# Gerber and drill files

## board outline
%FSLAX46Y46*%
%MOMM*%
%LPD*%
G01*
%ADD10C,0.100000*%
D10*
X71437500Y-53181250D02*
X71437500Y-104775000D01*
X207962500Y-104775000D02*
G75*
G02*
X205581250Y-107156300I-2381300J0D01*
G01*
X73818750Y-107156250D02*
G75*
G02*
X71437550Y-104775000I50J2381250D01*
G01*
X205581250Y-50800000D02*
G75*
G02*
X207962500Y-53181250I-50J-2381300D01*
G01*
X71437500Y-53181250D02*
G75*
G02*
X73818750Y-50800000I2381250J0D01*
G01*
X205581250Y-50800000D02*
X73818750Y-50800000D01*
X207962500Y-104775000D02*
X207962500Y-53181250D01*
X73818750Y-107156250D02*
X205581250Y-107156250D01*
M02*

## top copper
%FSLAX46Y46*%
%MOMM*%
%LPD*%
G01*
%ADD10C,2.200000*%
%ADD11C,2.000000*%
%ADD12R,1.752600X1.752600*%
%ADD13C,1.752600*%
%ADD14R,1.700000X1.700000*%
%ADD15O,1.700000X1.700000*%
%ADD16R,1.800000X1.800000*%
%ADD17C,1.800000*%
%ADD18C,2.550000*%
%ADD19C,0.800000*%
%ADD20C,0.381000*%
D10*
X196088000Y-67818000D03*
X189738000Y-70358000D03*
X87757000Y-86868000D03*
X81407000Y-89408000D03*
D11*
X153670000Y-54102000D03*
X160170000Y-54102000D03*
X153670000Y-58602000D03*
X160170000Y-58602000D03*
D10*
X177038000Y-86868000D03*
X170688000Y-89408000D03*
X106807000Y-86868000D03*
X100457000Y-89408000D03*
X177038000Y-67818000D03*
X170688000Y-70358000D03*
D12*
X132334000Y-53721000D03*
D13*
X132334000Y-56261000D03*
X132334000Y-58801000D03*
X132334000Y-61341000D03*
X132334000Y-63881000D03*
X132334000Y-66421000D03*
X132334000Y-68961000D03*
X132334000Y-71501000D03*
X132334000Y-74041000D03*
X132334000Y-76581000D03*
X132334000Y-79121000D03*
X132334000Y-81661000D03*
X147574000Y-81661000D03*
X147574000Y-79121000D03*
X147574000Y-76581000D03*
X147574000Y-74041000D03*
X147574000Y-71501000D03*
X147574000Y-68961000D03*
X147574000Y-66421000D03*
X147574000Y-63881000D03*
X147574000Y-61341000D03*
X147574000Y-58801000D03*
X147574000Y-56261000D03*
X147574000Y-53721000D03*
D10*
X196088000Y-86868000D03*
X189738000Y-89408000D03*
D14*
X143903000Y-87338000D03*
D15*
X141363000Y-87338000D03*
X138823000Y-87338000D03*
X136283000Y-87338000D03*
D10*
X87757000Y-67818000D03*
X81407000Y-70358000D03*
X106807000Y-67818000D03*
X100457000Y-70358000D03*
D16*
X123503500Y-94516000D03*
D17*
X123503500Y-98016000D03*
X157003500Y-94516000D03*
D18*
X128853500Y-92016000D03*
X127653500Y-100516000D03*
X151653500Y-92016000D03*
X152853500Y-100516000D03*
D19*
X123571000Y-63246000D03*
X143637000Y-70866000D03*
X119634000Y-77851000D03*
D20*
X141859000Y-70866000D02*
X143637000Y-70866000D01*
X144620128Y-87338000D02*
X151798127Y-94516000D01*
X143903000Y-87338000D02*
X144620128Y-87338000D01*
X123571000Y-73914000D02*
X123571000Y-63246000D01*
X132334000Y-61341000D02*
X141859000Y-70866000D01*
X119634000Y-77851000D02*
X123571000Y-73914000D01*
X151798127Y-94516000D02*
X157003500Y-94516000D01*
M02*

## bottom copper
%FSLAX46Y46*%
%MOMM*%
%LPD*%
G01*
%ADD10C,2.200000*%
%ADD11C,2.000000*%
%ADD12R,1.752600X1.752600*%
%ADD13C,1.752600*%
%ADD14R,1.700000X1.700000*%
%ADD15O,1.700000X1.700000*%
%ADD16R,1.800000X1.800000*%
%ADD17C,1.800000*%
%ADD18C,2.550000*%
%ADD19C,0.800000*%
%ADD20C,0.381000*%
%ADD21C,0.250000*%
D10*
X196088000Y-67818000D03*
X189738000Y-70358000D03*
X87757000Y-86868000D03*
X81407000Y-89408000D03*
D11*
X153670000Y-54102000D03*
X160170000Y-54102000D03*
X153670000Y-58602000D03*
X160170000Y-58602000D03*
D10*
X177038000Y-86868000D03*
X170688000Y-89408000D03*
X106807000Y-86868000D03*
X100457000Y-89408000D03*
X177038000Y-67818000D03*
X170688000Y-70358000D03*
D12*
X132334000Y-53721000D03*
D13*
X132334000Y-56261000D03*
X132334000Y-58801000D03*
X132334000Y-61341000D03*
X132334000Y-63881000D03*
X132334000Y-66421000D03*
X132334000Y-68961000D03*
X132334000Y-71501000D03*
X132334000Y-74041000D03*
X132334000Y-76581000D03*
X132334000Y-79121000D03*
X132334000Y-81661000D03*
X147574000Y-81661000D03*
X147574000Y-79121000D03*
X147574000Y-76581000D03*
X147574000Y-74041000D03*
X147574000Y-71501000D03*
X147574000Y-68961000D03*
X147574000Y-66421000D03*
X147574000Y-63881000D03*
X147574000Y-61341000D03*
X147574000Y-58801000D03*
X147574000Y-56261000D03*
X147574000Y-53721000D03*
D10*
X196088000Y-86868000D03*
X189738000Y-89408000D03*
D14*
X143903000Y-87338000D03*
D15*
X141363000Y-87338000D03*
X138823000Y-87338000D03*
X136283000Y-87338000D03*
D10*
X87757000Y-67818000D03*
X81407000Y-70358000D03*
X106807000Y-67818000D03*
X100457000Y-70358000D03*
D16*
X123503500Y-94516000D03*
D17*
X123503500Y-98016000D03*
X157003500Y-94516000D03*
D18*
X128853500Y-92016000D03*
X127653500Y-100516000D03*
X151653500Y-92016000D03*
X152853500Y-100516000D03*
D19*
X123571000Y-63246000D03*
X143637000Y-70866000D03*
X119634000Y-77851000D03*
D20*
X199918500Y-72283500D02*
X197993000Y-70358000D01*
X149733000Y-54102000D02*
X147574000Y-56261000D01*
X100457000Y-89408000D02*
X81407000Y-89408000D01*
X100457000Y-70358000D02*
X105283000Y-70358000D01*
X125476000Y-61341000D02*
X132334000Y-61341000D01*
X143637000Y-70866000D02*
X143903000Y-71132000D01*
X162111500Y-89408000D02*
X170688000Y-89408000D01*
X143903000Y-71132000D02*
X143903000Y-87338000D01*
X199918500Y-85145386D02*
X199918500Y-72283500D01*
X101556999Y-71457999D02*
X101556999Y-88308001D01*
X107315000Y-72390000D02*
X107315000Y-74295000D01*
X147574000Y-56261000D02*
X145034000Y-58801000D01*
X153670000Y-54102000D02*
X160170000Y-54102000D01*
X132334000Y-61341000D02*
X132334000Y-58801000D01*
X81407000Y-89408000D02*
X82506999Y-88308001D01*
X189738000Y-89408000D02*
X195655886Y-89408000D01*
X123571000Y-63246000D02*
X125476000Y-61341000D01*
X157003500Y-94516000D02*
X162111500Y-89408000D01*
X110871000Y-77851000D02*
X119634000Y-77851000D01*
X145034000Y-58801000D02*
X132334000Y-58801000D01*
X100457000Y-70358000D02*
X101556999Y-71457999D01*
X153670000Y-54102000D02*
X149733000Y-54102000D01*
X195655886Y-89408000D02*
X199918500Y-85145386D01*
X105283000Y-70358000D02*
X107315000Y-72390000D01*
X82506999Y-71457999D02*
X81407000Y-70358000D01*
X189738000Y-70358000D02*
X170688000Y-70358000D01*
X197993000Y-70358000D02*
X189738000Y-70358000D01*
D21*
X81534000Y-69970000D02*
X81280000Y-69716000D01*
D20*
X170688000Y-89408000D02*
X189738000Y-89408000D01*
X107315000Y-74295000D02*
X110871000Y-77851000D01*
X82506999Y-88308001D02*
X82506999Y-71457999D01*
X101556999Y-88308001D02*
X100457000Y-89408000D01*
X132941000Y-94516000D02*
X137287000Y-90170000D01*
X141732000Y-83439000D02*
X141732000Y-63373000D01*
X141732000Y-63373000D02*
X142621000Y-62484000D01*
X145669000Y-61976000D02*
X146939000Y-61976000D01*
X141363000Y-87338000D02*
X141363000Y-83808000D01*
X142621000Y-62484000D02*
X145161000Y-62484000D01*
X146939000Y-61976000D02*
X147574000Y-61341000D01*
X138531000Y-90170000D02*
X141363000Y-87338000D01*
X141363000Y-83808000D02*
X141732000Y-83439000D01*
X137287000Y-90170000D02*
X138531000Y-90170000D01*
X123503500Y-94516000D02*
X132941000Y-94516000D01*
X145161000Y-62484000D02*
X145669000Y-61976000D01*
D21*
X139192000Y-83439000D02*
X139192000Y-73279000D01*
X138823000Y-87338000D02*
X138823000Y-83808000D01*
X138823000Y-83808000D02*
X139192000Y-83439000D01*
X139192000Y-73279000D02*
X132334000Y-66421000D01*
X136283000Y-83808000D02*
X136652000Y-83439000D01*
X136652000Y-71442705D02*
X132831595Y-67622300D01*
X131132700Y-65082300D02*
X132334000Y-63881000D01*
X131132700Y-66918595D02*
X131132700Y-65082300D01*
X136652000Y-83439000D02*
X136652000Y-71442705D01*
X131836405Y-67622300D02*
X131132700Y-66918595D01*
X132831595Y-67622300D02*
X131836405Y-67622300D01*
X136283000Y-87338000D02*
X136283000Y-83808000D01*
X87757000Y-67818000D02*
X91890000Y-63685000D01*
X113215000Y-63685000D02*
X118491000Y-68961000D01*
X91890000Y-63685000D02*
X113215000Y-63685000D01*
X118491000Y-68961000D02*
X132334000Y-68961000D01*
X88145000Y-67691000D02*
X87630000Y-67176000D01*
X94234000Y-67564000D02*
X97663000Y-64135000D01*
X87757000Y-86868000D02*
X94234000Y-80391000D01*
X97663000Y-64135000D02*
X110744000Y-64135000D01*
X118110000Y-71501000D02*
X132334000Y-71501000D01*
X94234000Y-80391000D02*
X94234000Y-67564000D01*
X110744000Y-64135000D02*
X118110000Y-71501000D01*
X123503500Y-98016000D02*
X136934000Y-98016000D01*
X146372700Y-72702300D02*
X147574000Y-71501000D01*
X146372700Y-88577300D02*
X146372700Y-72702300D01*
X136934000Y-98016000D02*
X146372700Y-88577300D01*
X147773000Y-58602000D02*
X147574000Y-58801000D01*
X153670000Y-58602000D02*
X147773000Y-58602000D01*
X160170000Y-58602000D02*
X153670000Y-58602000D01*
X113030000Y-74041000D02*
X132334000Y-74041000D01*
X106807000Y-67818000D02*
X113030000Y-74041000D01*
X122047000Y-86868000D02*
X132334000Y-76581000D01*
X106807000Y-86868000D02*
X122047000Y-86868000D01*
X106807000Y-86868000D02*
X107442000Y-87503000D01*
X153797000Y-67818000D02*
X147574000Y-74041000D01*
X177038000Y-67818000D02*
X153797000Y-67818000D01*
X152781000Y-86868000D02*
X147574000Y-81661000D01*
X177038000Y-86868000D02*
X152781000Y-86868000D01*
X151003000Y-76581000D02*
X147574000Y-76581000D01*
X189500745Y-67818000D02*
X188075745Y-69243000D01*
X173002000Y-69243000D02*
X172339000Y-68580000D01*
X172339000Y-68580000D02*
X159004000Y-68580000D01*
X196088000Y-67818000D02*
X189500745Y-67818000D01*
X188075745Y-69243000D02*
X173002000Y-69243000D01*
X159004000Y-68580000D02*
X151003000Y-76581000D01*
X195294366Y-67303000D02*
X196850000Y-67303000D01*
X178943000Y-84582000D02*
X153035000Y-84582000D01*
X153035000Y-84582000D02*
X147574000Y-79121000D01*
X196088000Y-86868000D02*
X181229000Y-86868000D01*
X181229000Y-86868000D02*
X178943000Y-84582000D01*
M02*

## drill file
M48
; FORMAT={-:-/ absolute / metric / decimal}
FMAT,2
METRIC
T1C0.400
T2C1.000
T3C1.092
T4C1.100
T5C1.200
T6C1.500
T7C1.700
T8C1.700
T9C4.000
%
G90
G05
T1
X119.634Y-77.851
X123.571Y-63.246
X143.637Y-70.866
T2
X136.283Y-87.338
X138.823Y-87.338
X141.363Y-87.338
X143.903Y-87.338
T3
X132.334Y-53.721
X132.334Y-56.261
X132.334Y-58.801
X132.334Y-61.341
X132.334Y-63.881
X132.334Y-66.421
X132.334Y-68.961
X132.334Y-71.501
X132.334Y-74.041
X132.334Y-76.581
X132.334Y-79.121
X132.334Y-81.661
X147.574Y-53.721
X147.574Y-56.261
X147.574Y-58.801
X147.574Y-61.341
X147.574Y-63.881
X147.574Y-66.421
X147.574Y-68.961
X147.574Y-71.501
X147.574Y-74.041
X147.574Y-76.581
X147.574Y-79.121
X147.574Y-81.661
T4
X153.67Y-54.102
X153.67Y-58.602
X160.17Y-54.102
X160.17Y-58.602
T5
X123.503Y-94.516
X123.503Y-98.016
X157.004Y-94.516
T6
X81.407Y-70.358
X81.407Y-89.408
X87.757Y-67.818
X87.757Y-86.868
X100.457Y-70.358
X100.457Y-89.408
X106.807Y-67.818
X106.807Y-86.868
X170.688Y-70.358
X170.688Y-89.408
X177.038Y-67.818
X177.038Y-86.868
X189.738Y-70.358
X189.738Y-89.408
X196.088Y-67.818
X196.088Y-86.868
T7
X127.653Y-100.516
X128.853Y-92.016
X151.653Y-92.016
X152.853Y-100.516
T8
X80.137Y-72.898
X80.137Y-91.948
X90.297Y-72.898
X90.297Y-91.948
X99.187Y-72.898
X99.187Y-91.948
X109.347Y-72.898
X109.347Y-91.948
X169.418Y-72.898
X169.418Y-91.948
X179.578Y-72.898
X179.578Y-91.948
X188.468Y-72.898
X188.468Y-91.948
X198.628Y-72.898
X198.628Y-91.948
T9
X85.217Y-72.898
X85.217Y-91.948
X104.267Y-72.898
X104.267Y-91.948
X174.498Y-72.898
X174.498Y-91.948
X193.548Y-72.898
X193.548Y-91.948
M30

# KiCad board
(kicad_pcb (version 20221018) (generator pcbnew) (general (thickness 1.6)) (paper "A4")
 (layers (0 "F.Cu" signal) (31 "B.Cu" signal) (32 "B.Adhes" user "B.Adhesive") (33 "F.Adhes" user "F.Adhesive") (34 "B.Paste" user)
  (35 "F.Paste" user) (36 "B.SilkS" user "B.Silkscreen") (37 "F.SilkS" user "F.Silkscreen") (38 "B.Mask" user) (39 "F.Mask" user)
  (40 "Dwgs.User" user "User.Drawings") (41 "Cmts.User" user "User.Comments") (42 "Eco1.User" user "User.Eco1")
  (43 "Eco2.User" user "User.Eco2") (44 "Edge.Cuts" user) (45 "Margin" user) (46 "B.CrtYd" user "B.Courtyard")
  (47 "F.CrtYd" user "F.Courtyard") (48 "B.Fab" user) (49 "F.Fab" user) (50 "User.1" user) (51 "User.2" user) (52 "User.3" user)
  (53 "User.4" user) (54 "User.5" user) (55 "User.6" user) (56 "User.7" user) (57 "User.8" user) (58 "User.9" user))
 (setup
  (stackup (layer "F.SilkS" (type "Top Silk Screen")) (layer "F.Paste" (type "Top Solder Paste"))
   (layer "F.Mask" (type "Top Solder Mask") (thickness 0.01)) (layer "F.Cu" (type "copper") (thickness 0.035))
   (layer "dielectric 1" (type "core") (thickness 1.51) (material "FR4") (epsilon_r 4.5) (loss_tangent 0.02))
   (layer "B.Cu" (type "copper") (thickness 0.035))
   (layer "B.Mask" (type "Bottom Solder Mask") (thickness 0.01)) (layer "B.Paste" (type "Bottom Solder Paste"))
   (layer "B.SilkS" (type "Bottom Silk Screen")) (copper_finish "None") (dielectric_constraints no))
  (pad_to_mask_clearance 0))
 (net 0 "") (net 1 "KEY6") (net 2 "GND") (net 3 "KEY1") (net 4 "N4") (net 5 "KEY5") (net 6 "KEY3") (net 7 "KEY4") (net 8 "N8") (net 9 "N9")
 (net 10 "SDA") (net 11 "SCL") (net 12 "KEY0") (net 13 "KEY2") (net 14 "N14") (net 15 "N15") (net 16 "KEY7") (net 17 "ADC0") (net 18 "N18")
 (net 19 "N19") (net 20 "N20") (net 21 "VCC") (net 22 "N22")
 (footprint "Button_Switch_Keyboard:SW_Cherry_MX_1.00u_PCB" (layer "F.Cu") (at 196.088 67.818)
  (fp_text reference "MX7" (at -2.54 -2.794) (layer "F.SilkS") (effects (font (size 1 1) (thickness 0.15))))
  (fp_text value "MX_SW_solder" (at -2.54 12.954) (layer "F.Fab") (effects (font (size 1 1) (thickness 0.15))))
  (pad "" np_thru_hole circle (at -7.62 5.08) (size 1.7 1.7) (drill 1.7) (layers "*.Cu" "*.Mask"))
  (pad "" np_thru_hole circle (at -2.54 5.08) (size 4 4) (drill 4) (layers "*.Cu" "*.Mask"))
  (pad "" np_thru_hole circle (at 2.54 5.08) (size 1.7 1.7) (drill 1.7) (layers "*.Cu" "*.Mask"))
  (pad "1" thru_hole circle (at 0 0) (size 2.2 2.2) (drill 1.5) (layers "*.Cu" "*.Mask") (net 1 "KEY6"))
  (pad "2" thru_hole circle (at -6.35 2.54) (size 2.2 2.2) (drill 1.5) (layers "*.Cu" "*.Mask") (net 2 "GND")))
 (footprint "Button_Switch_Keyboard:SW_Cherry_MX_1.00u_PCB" (layer "F.Cu") (at 87.757 86.868)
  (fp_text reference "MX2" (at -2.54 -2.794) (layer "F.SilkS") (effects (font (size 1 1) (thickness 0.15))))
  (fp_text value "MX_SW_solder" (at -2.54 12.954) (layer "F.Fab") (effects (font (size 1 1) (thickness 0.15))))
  (pad "" np_thru_hole circle (at -7.62 5.08) (size 1.7 1.7) (drill 1.7) (layers "*.Cu" "*.Mask"))
  (pad "" np_thru_hole circle (at -2.54 5.08) (size 4 4) (drill 4) (layers "*.Cu" "*.Mask"))
  (pad "" np_thru_hole circle (at 2.54 5.08) (size 1.7 1.7) (drill 1.7) (layers "*.Cu" "*.Mask"))
  (pad "1" thru_hole circle (at 0 0) (size 2.2 2.2) (drill 1.5) (layers "*.Cu" "*.Mask") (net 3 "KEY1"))
  (pad "2" thru_hole circle (at -6.35 2.54) (size 2.2 2.2) (drill 1.5) (layers "*.Cu" "*.Mask") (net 2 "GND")))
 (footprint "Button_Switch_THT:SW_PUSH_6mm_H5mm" (layer "F.Cu") (at 153.67 54.102)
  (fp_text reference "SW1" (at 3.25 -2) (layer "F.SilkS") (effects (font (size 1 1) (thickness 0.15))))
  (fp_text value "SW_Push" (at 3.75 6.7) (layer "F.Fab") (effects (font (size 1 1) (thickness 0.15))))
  (pad "1" thru_hole circle (at 0 0 90) (size 2 2) (drill 1.1) (layers "*.Cu" "*.Mask") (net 2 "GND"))
  (pad "1" thru_hole circle (at 6.5 0 90) (size 2 2) (drill 1.1) (layers "*.Cu" "*.Mask") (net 2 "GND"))
  (pad "2" thru_hole circle (at 0 4.5 90) (size 2 2) (drill 1.1) (layers "*.Cu" "*.Mask") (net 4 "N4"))
  (pad "2" thru_hole circle (at 6.5 4.5 90) (size 2 2) (drill 1.1) (layers "*.Cu" "*.Mask") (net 4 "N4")))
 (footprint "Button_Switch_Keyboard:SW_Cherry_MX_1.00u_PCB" (layer "F.Cu") (at 177.038 86.868)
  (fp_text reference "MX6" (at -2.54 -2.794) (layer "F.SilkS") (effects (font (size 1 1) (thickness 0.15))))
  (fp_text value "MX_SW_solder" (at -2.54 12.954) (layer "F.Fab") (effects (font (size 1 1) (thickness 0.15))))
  (pad "" np_thru_hole circle (at -7.62 5.08) (size 1.7 1.7) (drill 1.7) (layers "*.Cu" "*.Mask"))
  (pad "" np_thru_hole circle (at -2.54 5.08) (size 4 4) (drill 4) (layers "*.Cu" "*.Mask"))
  (pad "" np_thru_hole circle (at 2.54 5.08) (size 1.7 1.7) (drill 1.7) (layers "*.Cu" "*.Mask"))
  (pad "1" thru_hole circle (at 0 0) (size 2.2 2.2) (drill 1.5) (layers "*.Cu" "*.Mask") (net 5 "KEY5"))
  (pad "2" thru_hole circle (at -6.35 2.54) (size 2.2 2.2) (drill 1.5) (layers "*.Cu" "*.Mask") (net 2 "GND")))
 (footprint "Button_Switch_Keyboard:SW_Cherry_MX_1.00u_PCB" (layer "F.Cu") (at 106.807 86.868)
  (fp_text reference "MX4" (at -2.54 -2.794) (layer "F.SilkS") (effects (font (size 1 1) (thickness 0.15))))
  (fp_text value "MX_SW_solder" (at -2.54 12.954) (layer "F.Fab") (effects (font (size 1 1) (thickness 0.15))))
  (pad "" np_thru_hole circle (at -7.62 5.08) (size 1.7 1.7) (drill 1.7) (layers "*.Cu" "*.Mask"))
  (pad "" np_thru_hole circle (at -2.54 5.08) (size 4 4) (drill 4) (layers "*.Cu" "*.Mask"))
  (pad "" np_thru_hole circle (at 2.54 5.08) (size 1.7 1.7) (drill 1.7) (layers "*.Cu" "*.Mask"))
  (pad "1" thru_hole circle (at 0 0) (size 2.2 2.2) (drill 1.5) (layers "*.Cu" "*.Mask") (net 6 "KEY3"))
  (pad "2" thru_hole circle (at -6.35 2.54) (size 2.2 2.2) (drill 1.5) (layers "*.Cu" "*.Mask") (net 2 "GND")))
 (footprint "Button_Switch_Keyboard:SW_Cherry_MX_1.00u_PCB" (layer "F.Cu") (at 177.038 67.818)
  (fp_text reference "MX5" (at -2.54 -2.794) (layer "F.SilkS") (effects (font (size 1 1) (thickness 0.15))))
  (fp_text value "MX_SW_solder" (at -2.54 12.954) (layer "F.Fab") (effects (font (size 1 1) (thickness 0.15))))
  (pad "" np_thru_hole circle (at -7.62 5.08) (size 1.7 1.7) (drill 1.7) (layers "*.Cu" "*.Mask"))
  (pad "" np_thru_hole circle (at -2.54 5.08) (size 4 4) (drill 4) (layers "*.Cu" "*.Mask"))
  (pad "" np_thru_hole circle (at 2.54 5.08) (size 1.7 1.7) (drill 1.7) (layers "*.Cu" "*.Mask"))
  (pad "1" thru_hole circle (at 0 0) (size 2.2 2.2) (drill 1.5) (layers "*.Cu" "*.Mask") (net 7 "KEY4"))
  (pad "2" thru_hole circle (at -6.35 2.54) (size 2.2 2.2) (drill 1.5) (layers "*.Cu" "*.Mask") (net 2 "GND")))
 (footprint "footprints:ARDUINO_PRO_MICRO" (layer "F.Cu") (at 139.954 67.691 -90)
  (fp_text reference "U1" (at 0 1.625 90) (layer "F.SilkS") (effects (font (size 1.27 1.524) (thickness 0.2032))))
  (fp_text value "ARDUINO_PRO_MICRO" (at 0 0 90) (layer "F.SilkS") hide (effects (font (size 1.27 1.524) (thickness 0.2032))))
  (pad "1" thru_hole rect (at -13.97 7.62 270) (size 1.7526 1.7526) (drill 1.0922) (layers "*.Cu" "*.SilkS" "*.Mask") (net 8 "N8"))
  (pad "2" thru_hole circle (at -11.43 7.62 270) (size 1.7526 1.7526) (drill 1.0922) (layers "*.Cu" "*.SilkS" "*.Mask") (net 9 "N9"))
  (pad "3" thru_hole circle (at -8.89 7.62 270) (size 1.7526 1.7526) (drill 1.0922) (layers "*.Cu" "*.SilkS" "*.Mask") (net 2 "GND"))
  (pad "4" thru_hole circle (at -6.35 7.62 270) (size 1.7526 1.7526) (drill 1.0922) (layers "*.Cu" "*.SilkS" "*.Mask") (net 2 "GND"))
  (pad "5" thru_hole circle (at -3.81 7.62 270) (size 1.7526 1.7526) (drill 1.0922) (layers "*.Cu" "*.SilkS" "*.Mask") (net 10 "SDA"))
  (pad "6" thru_hole circle (at -1.27 7.62 270) (size 1.7526 1.7526) (drill 1.0922) (layers "*.Cu" "*.SilkS" "*.Mask") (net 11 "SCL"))
  (pad "7" thru_hole circle (at 1.27 7.62 270) (size 1.7526 1.7526) (drill 1.0922) (layers "*.Cu" "*.SilkS" "*.Mask") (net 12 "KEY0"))
  (pad "8" thru_hole circle (at 3.81 7.62 270) (size 1.7526 1.7526) (drill 1.0922) (layers "*.Cu" "*.SilkS" "*.Mask") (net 3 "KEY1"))
  (pad "9" thru_hole circle (at 6.35 7.62 270) (size 1.7526 1.7526) (drill 1.0922) (layers "*.Cu" "*.SilkS" "*.Mask") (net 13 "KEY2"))
  (pad "10" thru_hole circle (at 8.89 7.62 270) (size 1.7526 1.7526) (drill 1.0922) (layers "*.Cu" "*.SilkS" "*.Mask") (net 6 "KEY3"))
  (pad "11" thru_hole circle (at 11.43 7.62 270) (size 1.7526 1.7526) (drill 1.0922) (layers "*.Cu" "*.SilkS" "*.Mask") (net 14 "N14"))
  (pad "12" thru_hole circle (at 13.97 7.62 270) (size 1.7526 1.7526) (drill 1.0922) (layers "*.Cu" "*.SilkS" "*.Mask") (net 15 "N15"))
  (pad "13" thru_hole circle (at 13.97 -7.62 270) (size 1.7526 1.7526) (drill 1.0922) (layers "*.Cu" "*.SilkS" "*.Mask") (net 5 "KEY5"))
  (pad "14" thru_hole circle (at 11.43 -7.62 270) (size 1.7526 1.7526) (drill 1.0922) (layers "*.Cu" "*.SilkS" "*.Mask") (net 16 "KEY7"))
  (pad "15" thru_hole circle (at 8.89 -7.62 270) (size 1.7526 1.7526) (drill 1.0922) (layers "*.Cu" "*.SilkS" "*.Mask") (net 1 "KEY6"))
  (pad "16" thru_hole circle (at 6.35 -7.62 270) (size 1.7526 1.7526) (drill 1.0922) (layers "*.Cu" "*.SilkS" "*.Mask") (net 7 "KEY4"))
  (pad "17" thru_hole circle (at 3.81 -7.62 270) (size 1.7526 1.7526) (drill 1.0922) (layers "*.Cu" "*.SilkS" "*.Mask") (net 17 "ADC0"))
  (pad "18" thru_hole circle (at 1.27 -7.62 270) (size 1.7526 1.7526) (drill 1.0922) (layers "*.Cu" "*.SilkS" "*.Mask") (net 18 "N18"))
  (pad "19" thru_hole circle (at -1.27 -7.62 270) (size 1.7526 1.7526) (drill 1.0922) (layers "*.Cu" "*.SilkS" "*.Mask") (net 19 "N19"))
  (pad "20" thru_hole circle (at -3.81 -7.62 270) (size 1.7526 1.7526) (drill 1.0922) (layers "*.Cu" "*.SilkS" "*.Mask") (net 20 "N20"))
  (pad "21" thru_hole circle (at -6.35 -7.62 270) (size 1.7526 1.7526) (drill 1.0922) (layers "*.Cu" "*.SilkS" "*.Mask") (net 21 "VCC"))
  (pad "22" thru_hole circle (at -8.89 -7.62 270) (size 1.7526 1.7526) (drill 1.0922) (layers "*.Cu" "*.SilkS" "*.Mask") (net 4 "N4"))
  (pad "23" thru_hole circle (at -11.43 -7.62 270) (size 1.7526 1.7526) (drill 1.0922) (layers "*.Cu" "*.SilkS" "*.Mask") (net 2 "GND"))
  (pad "24" thru_hole circle (at -13.97 -7.62 270) (size 1.7526 1.7526) (drill 1.0922) (layers "*.Cu" "*.SilkS" "*.Mask") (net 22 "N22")))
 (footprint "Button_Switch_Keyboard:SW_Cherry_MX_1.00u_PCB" (layer "F.Cu") (at 196.088 86.868)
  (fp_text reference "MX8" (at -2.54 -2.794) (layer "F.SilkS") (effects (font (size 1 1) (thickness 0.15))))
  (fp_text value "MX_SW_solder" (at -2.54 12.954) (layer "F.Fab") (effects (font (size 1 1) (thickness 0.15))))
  (pad "" np_thru_hole circle (at -7.62 5.08) (size 1.7 1.7) (drill 1.7) (layers "*.Cu" "*.Mask"))
  (pad "" np_thru_hole circle (at -2.54 5.08) (size 4 4) (drill 4) (layers "*.Cu" "*.Mask"))
  (pad "" np_thru_hole circle (at 2.54 5.08) (size 1.7 1.7) (drill 1.7) (layers "*.Cu" "*.Mask"))
  (pad "1" thru_hole circle (at 0 0) (size 2.2 2.2) (drill 1.5) (layers "*.Cu" "*.Mask") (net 16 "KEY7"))
  (pad "2" thru_hole circle (at -6.35 2.54) (size 2.2 2.2) (drill 1.5) (layers "*.Cu" "*.Mask") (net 2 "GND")))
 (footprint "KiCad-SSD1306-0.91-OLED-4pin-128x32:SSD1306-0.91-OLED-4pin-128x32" (layer "F.Cu") (at 146.093 50.838 -90)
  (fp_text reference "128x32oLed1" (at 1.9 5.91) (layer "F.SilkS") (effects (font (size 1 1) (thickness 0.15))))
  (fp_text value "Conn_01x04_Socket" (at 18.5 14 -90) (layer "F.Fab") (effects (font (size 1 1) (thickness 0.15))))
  (pad "1" thru_hole rect (at 36.5 2.19 270) (size 1.7 1.7) (drill 1) (layers "*.Cu" "*.Mask") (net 2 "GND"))
  (pad "2" thru_hole oval (at 36.5 4.73 270) (size 1.7 1.7) (drill 1) (layers "*.Cu" "*.Mask") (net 21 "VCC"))
  (pad "3" thru_hole oval (at 36.5 7.27 270) (size 1.7 1.7) (drill 1) (layers "*.Cu" "*.Mask") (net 11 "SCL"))
  (pad "4" thru_hole oval (at 36.5 9.81 270) (size 1.7 1.7) (drill 1) (layers "*.Cu" "*.Mask") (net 10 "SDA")))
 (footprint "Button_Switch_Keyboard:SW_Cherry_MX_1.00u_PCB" (layer "F.Cu") (at 87.757 67.818)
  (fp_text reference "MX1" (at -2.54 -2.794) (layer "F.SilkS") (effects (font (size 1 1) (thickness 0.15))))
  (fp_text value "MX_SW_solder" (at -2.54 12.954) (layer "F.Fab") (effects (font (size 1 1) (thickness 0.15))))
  (pad "" np_thru_hole circle (at -7.62 5.08) (size 1.7 1.7) (drill 1.7) (layers "*.Cu" "*.Mask"))
  (pad "" np_thru_hole circle (at -2.54 5.08) (size 4 4) (drill 4) (layers "*.Cu" "*.Mask"))
  (pad "" np_thru_hole circle (at 2.54 5.08) (size 1.7 1.7) (drill 1.7) (layers "*.Cu" "*.Mask"))
  (pad "1" thru_hole circle (at 0 0) (size 2.2 2.2) (drill 1.5) (layers "*.Cu" "*.Mask") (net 12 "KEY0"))
  (pad "2" thru_hole circle (at -6.35 2.54) (size 2.2 2.2) (drill 1.5) (layers "*.Cu" "*.Mask") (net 2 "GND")))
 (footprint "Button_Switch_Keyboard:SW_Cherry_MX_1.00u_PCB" (layer "F.Cu") (at 106.807 67.818)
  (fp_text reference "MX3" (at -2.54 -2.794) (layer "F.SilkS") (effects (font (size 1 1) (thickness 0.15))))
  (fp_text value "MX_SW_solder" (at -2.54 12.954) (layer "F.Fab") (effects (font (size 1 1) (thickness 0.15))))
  (pad "" np_thru_hole circle (at -7.62 5.08) (size 1.7 1.7) (drill 1.7) (layers "*.Cu" "*.Mask"))
  (pad "" np_thru_hole circle (at -2.54 5.08) (size 4 4) (drill 4) (layers "*.Cu" "*.Mask"))
  (pad "" np_thru_hole circle (at 2.54 5.08) (size 1.7 1.7) (drill 1.7) (layers "*.Cu" "*.Mask"))
  (pad "1" thru_hole circle (at 0 0) (size 2.2 2.2) (drill 1.5) (layers "*.Cu" "*.Mask") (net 13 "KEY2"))
  (pad "2" thru_hole circle (at -6.35 2.54) (size 2.2 2.2) (drill 1.5) (layers "*.Cu" "*.Mask") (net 2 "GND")))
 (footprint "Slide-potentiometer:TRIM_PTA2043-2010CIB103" (layer "F.Cu") (at 140.2535 96.266)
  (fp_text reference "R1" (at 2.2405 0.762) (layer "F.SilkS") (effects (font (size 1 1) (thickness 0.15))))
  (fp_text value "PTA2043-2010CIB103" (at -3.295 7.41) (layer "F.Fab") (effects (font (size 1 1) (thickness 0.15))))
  (pad "1" thru_hole rect (at -16.75 -1.75) (size 1.8 1.8) (drill 1.2) (layers "*.Cu" "*.Mask") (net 21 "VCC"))
  (pad "2" thru_hole circle (at -16.75 1.75) (size 1.8 1.8) (drill 1.2) (layers "*.Cu" "*.Mask") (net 17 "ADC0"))
  (pad "3" thru_hole circle (at 16.75 -1.75) (size 1.8 1.8) (drill 1.2) (layers "*.Cu" "*.Mask") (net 2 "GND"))
  (pad "S1" thru_hole circle (at -11.4 -4.25) (size 2.55 2.55) (drill 1.7) (layers "*.Cu" "*.Mask"))
  (pad "S2" thru_hole circle (at -12.6 4.25) (size 2.55 2.55) (drill 1.7) (layers "*.Cu" "*.Mask"))
  (pad "S3" thru_hole circle (at 11.4 -4.25) (size 2.55 2.55) (drill 1.7) (layers "*.Cu" "*.Mask"))
  (pad "S4" thru_hole circle (at 12.6 4.25) (size 2.55 2.55) (drill 1.7) (layers "*.Cu" "*.Mask")))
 (gr_line (start 71.4375 53.18125) (end 71.4375 104.775) (stroke (width 0.1) (type default)) (layer "Edge.Cuts"))
 (gr_arc (start 207.9625 104.775) (mid 207.265048 106.458798) (end 205.58125 107.15625) (stroke (width 0.1) (type default))
  (layer "Edge.Cuts"))
 (gr_arc (start 73.81875 107.15625) (mid 72.134952 106.458798) (end 71.4375 104.775) (stroke (width 0.1) (type default)) (layer "Edge.Cuts"))
 (gr_arc (start 205.58125 50.8) (mid 207.265048 51.497452) (end 207.9625 53.18125) (stroke (width 0.1) (type default)) (layer "Edge.Cuts"))
 (gr_arc (start 71.4375 53.18125) (mid 72.134952 51.497452) (end 73.81875 50.8) (stroke (width 0.1) (type default)) (layer "Edge.Cuts"))
 (gr_line (start 205.58125 50.8) (end 73.81875 50.8) (stroke (width 0.1) (type default)) (layer "Edge.Cuts"))
 (gr_line (start 207.9625 104.775) (end 207.9625 53.18125) (stroke (width 0.1) (type default)) (layer "Edge.Cuts"))
 (gr_line (start 73.81875 107.15625) (end 205.58125 107.15625) (stroke (width 0.1) (type default)) (layer "Edge.Cuts"))
 (segment (start 141.859 70.866) (end 143.637 70.866) (width 0.381) (layer "F.Cu") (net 2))
 (segment (start 144.620128 87.338) (end 151.798127 94.516) (width 0.381) (layer "F.Cu") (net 2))
 (segment (start 143.903 87.338) (end 144.620128 87.338) (width 0.381) (layer "F.Cu") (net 2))
 (segment (start 123.571 73.914) (end 123.571 63.246) (width 0.381) (layer "F.Cu") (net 2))
 (segment (start 132.334 61.341) (end 141.859 70.866) (width 0.381) (layer "F.Cu") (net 2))
 (segment (start 119.634 77.851) (end 123.571 73.914) (width 0.381) (layer "F.Cu") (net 2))
 (segment (start 151.798127 94.516) (end 157.0035 94.516) (width 0.381) (layer "F.Cu") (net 2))
 (via (at 123.571 63.246) (size 0.8) (drill 0.4) (layers "F.Cu" "B.Cu") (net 2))
 (via (at 143.637 70.866) (size 0.8) (drill 0.4) (layers "F.Cu" "B.Cu") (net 2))
 (via (at 119.634 77.851) (size 0.8) (drill 0.4) (layers "F.Cu" "B.Cu") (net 2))
 (segment (start 199.9185 72.2835) (end 197.993 70.358) (width 0.381) (layer "B.Cu") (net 2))
 (segment (start 149.733 54.102) (end 147.574 56.261) (width 0.381) (layer "B.Cu") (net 2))
 (segment (start 100.457 89.408) (end 81.407 89.408) (width 0.381) (layer "B.Cu") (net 2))
 (segment (start 100.457 70.358) (end 105.283 70.358) (width 0.381) (layer "B.Cu") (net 2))
 (segment (start 125.476 61.341) (end 132.334 61.341) (width 0.381) (layer "B.Cu") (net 2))
 (segment (start 143.637 70.866) (end 143.903 71.132) (width 0.381) (layer "B.Cu") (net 2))
 (segment (start 162.1115 89.408) (end 170.688 89.408) (width 0.381) (layer "B.Cu") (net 2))
 (segment (start 143.903 71.132) (end 143.903 87.338) (width 0.381) (layer "B.Cu") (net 2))
 (segment (start 199.9185 85.145386) (end 199.9185 72.2835) (width 0.381) (layer "B.Cu") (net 2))
 (segment (start 101.556999 71.457999) (end 101.556999 88.308001) (width 0.381) (layer "B.Cu") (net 2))
 (segment (start 107.315 72.39) (end 107.315 74.295) (width 0.381) (layer "B.Cu") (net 2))
 (segment (start 147.574 56.261) (end 145.034 58.801) (width 0.381) (layer "B.Cu") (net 2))
 (segment (start 153.67 54.102) (end 160.17 54.102) (width 0.381) (layer "B.Cu") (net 2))
 (segment (start 132.334 61.341) (end 132.334 58.801) (width 0.381) (layer "B.Cu") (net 2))
 (segment (start 81.407 89.408) (end 82.506999 88.308001) (width 0.381) (layer "B.Cu") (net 2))
 (segment (start 189.738 89.408) (end 195.655886 89.408) (width 0.381) (layer "B.Cu") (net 2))
 (segment (start 123.571 63.246) (end 125.476 61.341) (width 0.381) (layer "B.Cu") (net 2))
 (segment (start 157.0035 94.516) (end 162.1115 89.408) (width 0.381) (layer "B.Cu") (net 2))
 (segment (start 110.871 77.851) (end 119.634 77.851) (width 0.381) (layer "B.Cu") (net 2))
 (segment (start 145.034 58.801) (end 132.334 58.801) (width 0.381) (layer "B.Cu") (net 2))
 (segment (start 100.457 70.358) (end 101.556999 71.457999) (width 0.381) (layer "B.Cu") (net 2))
 (segment (start 153.67 54.102) (end 149.733 54.102) (width 0.381) (layer "B.Cu") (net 2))
 (segment (start 195.655886 89.408) (end 199.9185 85.145386) (width 0.381) (layer "B.Cu") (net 2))
 (segment (start 105.283 70.358) (end 107.315 72.39) (width 0.381) (layer "B.Cu") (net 2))
 (segment (start 82.506999 71.457999) (end 81.407 70.358) (width 0.381) (layer "B.Cu") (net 2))
 (segment (start 189.738 70.358) (end 170.688 70.358) (width 0.381) (layer "B.Cu") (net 2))
 (segment (start 197.993 70.358) (end 189.738 70.358) (width 0.381) (layer "B.Cu") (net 2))
 (segment (start 81.534 69.97) (end 81.28 69.716) (width 0.25) (layer "B.Cu") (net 2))
 (segment (start 170.688 89.408) (end 189.738 89.408) (width 0.381) (layer "B.Cu") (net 2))
 (segment (start 107.315 74.295) (end 110.871 77.851) (width 0.381) (layer "B.Cu") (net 2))
 (segment (start 82.506999 88.308001) (end 82.506999 71.457999) (width 0.381) (layer "B.Cu") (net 2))
 (segment (start 101.556999 88.308001) (end 100.457 89.408) (width 0.381) (layer "B.Cu") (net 2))
 (segment (start 132.941 94.516) (end 137.287 90.17) (width 0.381) (layer "B.Cu") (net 21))
 (segment (start 141.732 83.439) (end 141.732 63.373) (width 0.381) (layer "B.Cu") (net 21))
 (segment (start 141.732 63.373) (end 142.621 62.484) (width 0.381) (layer "B.Cu") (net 21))
 (segment (start 145.669 61.976) (end 146.939 61.976) (width 0.381) (layer "B.Cu") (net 21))
 (segment (start 141.363 87.338) (end 141.363 83.808) (width 0.381) (layer "B.Cu") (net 21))
 (segment (start 142.621 62.484) (end 145.161 62.484) (width 0.381) (layer "B.Cu") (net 21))
 (segment (start 146.939 61.976) (end 147.574 61.341) (width 0.381) (layer "B.Cu") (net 21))
 (segment (start 138.531 90.17) (end 141.363 87.338) (width 0.381) (layer "B.Cu") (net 21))
 (segment (start 141.363 83.808) (end 141.732 83.439) (width 0.381) (layer "B.Cu") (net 21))
 (segment (start 137.287 90.17) (end 138.531 90.17) (width 0.381) (layer "B.Cu") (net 21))
 (segment (start 123.5035 94.516) (end 132.941 94.516) (width 0.381) (layer "B.Cu") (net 21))
 (segment (start 145.161 62.484) (end 145.669 61.976) (width 0.381) (layer "B.Cu") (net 21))
 (segment (start 139.192 83.439) (end 139.192 73.279) (width 0.25) (layer "B.Cu") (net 11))
 (segment (start 138.823 87.338) (end 138.823 83.808) (width 0.25) (layer "B.Cu") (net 11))
 (segment (start 138.823 83.808) (end 139.192 83.439) (width 0.25) (layer "B.Cu") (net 11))
 (segment (start 139.192 73.279) (end 132.334 66.421) (width 0.25) (layer "B.Cu") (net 11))
 (segment (start 136.283 83.808) (end 136.652 83.439) (width 0.25) (layer "B.Cu") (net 10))
 (segment (start 136.652 71.442705) (end 132.831595 67.6223) (width 0.25) (layer "B.Cu") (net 10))
 (segment (start 131.1327 65.0823) (end 132.334 63.881) (width 0.25) (layer "B.Cu") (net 10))
 (segment (start 131.1327 66.918595) (end 131.1327 65.0823) (width 0.25) (layer "B.Cu") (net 10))
 (segment (start 136.652 83.439) (end 136.652 71.442705) (width 0.25) (layer "B.Cu") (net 10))
 (segment (start 131.836405 67.6223) (end 131.1327 66.918595) (width 0.25) (layer "B.Cu") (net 10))
 (segment (start 132.831595 67.6223) (end 131.836405 67.6223) (width 0.25) (layer "B.Cu") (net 10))
 (segment (start 136.283 87.338) (end 136.283 83.808) (width 0.25) (layer "B.Cu") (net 10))
 (segment (start 87.757 67.818) (end 91.89 63.685) (width 0.25) (layer "B.Cu") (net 12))
 (segment (start 113.215 63.685) (end 118.491 68.961) (width 0.25) (layer "B.Cu") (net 12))
 (segment (start 91.89 63.685) (end 113.215 63.685) (width 0.25) (layer "B.Cu") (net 12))
 (segment (start 118.491 68.961) (end 132.334 68.961) (width 0.25) (layer "B.Cu") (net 12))
 (segment (start 88.145 67.691) (end 87.63 67.176) (width 0.25) (layer "B.Cu") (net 12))
 (segment (start 94.234 67.564) (end 97.663 64.135) (width 0.25) (layer "B.Cu") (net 3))
 (segment (start 87.757 86.868) (end 94.234 80.391) (width 0.25) (layer "B.Cu") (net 3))
 (segment (start 97.663 64.135) (end 110.744 64.135) (width 0.25) (layer "B.Cu") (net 3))
 (segment (start 118.11 71.501) (end 132.334 71.501) (width 0.25) (layer "B.Cu") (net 3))
 (segment (start 94.234 80.391) (end 94.234 67.564) (width 0.25) (layer "B.Cu") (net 3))
 (segment (start 110.744 64.135) (end 118.11 71.501) (width 0.25) (layer "B.Cu") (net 3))
 (segment (start 123.5035 98.016) (end 136.934 98.016) (width 0.25) (layer "B.Cu") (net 17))
 (segment (start 146.3727 72.7023) (end 147.574 71.501) (width 0.25) (layer "B.Cu") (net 17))
 (segment (start 146.3727 88.5773) (end 146.3727 72.7023) (width 0.25) (layer "B.Cu") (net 17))
 (segment (start 136.934 98.016) (end 146.3727 88.5773) (width 0.25) (layer "B.Cu") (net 17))
 (segment (start 147.773 58.602) (end 147.574 58.801) (width 0.25) (layer "B.Cu") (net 4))
 (segment (start 153.67 58.602) (end 147.773 58.602) (width 0.25) (layer "B.Cu") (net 4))
 (segment (start 160.17 58.602) (end 153.67 58.602) (width 0.25) (layer "B.Cu") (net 4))
 (segment (start 113.03 74.041) (end 132.334 74.041) (width 0.25) (layer "B.Cu") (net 13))
 (segment (start 106.807 67.818) (end 113.03 74.041) (width 0.25) (layer "B.Cu") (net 13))
 (segment (start 122.047 86.868) (end 132.334 76.581) (width 0.25) (layer "B.Cu") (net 6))
 (segment (start 106.807 86.868) (end 122.047 86.868) (width 0.25) (layer "B.Cu") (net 6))
 (segment (start 106.807 86.868) (end 107.442 87.503) (width 0.25) (layer "B.Cu") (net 6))
 (segment (start 153.797 67.818) (end 147.574 74.041) (width 0.25) (layer "B.Cu") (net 7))
 (segment (start 177.038 67.818) (end 153.797 67.818) (width 0.25) (layer "B.Cu") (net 7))
 (segment (start 152.781 86.868) (end 147.574 81.661) (width 0.25) (layer "B.Cu") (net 5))
 (segment (start 177.038 86.868) (end 152.781 86.868) (width 0.25) (layer "B.Cu") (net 5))
 (segment (start 151.003 76.581) (end 147.574 76.581) (width 0.25) (layer "B.Cu") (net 1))
 (segment (start 189.500745 67.818) (end 188.075745 69.243) (width 0.25) (layer "B.Cu") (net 1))
 (segment (start 173.002 69.243) (end 172.339 68.58) (width 0.25) (layer "B.Cu") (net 1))
 (segment (start 172.339 68.58) (end 159.004 68.58) (width 0.25) (layer "B.Cu") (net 1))
 (segment (start 196.088 67.818) (end 189.500745 67.818) (width 0.25) (layer "B.Cu") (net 1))
 (segment (start 188.075745 69.243) (end 173.002 69.243) (width 0.25) (layer "B.Cu") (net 1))
 (segment (start 159.004 68.58) (end 151.003 76.581) (width 0.25) (layer "B.Cu") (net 1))
 (segment (start 195.294366 67.303) (end 196.85 67.303) (width 0.25) (layer "B.Cu") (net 1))
 (segment (start 178.943 84.582) (end 153.035 84.582) (width 0.25) (layer "B.Cu") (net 16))
 (segment (start 153.035 84.582) (end 147.574 79.121) (width 0.25) (layer "B.Cu") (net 16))
 (segment (start 196.088 86.868) (end 181.229 86.868) (width 0.25) (layer "B.Cu") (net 16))
 (segment (start 181.229 86.868) (end 178.943 84.582) (width 0.25) (layer "B.Cu") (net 16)))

